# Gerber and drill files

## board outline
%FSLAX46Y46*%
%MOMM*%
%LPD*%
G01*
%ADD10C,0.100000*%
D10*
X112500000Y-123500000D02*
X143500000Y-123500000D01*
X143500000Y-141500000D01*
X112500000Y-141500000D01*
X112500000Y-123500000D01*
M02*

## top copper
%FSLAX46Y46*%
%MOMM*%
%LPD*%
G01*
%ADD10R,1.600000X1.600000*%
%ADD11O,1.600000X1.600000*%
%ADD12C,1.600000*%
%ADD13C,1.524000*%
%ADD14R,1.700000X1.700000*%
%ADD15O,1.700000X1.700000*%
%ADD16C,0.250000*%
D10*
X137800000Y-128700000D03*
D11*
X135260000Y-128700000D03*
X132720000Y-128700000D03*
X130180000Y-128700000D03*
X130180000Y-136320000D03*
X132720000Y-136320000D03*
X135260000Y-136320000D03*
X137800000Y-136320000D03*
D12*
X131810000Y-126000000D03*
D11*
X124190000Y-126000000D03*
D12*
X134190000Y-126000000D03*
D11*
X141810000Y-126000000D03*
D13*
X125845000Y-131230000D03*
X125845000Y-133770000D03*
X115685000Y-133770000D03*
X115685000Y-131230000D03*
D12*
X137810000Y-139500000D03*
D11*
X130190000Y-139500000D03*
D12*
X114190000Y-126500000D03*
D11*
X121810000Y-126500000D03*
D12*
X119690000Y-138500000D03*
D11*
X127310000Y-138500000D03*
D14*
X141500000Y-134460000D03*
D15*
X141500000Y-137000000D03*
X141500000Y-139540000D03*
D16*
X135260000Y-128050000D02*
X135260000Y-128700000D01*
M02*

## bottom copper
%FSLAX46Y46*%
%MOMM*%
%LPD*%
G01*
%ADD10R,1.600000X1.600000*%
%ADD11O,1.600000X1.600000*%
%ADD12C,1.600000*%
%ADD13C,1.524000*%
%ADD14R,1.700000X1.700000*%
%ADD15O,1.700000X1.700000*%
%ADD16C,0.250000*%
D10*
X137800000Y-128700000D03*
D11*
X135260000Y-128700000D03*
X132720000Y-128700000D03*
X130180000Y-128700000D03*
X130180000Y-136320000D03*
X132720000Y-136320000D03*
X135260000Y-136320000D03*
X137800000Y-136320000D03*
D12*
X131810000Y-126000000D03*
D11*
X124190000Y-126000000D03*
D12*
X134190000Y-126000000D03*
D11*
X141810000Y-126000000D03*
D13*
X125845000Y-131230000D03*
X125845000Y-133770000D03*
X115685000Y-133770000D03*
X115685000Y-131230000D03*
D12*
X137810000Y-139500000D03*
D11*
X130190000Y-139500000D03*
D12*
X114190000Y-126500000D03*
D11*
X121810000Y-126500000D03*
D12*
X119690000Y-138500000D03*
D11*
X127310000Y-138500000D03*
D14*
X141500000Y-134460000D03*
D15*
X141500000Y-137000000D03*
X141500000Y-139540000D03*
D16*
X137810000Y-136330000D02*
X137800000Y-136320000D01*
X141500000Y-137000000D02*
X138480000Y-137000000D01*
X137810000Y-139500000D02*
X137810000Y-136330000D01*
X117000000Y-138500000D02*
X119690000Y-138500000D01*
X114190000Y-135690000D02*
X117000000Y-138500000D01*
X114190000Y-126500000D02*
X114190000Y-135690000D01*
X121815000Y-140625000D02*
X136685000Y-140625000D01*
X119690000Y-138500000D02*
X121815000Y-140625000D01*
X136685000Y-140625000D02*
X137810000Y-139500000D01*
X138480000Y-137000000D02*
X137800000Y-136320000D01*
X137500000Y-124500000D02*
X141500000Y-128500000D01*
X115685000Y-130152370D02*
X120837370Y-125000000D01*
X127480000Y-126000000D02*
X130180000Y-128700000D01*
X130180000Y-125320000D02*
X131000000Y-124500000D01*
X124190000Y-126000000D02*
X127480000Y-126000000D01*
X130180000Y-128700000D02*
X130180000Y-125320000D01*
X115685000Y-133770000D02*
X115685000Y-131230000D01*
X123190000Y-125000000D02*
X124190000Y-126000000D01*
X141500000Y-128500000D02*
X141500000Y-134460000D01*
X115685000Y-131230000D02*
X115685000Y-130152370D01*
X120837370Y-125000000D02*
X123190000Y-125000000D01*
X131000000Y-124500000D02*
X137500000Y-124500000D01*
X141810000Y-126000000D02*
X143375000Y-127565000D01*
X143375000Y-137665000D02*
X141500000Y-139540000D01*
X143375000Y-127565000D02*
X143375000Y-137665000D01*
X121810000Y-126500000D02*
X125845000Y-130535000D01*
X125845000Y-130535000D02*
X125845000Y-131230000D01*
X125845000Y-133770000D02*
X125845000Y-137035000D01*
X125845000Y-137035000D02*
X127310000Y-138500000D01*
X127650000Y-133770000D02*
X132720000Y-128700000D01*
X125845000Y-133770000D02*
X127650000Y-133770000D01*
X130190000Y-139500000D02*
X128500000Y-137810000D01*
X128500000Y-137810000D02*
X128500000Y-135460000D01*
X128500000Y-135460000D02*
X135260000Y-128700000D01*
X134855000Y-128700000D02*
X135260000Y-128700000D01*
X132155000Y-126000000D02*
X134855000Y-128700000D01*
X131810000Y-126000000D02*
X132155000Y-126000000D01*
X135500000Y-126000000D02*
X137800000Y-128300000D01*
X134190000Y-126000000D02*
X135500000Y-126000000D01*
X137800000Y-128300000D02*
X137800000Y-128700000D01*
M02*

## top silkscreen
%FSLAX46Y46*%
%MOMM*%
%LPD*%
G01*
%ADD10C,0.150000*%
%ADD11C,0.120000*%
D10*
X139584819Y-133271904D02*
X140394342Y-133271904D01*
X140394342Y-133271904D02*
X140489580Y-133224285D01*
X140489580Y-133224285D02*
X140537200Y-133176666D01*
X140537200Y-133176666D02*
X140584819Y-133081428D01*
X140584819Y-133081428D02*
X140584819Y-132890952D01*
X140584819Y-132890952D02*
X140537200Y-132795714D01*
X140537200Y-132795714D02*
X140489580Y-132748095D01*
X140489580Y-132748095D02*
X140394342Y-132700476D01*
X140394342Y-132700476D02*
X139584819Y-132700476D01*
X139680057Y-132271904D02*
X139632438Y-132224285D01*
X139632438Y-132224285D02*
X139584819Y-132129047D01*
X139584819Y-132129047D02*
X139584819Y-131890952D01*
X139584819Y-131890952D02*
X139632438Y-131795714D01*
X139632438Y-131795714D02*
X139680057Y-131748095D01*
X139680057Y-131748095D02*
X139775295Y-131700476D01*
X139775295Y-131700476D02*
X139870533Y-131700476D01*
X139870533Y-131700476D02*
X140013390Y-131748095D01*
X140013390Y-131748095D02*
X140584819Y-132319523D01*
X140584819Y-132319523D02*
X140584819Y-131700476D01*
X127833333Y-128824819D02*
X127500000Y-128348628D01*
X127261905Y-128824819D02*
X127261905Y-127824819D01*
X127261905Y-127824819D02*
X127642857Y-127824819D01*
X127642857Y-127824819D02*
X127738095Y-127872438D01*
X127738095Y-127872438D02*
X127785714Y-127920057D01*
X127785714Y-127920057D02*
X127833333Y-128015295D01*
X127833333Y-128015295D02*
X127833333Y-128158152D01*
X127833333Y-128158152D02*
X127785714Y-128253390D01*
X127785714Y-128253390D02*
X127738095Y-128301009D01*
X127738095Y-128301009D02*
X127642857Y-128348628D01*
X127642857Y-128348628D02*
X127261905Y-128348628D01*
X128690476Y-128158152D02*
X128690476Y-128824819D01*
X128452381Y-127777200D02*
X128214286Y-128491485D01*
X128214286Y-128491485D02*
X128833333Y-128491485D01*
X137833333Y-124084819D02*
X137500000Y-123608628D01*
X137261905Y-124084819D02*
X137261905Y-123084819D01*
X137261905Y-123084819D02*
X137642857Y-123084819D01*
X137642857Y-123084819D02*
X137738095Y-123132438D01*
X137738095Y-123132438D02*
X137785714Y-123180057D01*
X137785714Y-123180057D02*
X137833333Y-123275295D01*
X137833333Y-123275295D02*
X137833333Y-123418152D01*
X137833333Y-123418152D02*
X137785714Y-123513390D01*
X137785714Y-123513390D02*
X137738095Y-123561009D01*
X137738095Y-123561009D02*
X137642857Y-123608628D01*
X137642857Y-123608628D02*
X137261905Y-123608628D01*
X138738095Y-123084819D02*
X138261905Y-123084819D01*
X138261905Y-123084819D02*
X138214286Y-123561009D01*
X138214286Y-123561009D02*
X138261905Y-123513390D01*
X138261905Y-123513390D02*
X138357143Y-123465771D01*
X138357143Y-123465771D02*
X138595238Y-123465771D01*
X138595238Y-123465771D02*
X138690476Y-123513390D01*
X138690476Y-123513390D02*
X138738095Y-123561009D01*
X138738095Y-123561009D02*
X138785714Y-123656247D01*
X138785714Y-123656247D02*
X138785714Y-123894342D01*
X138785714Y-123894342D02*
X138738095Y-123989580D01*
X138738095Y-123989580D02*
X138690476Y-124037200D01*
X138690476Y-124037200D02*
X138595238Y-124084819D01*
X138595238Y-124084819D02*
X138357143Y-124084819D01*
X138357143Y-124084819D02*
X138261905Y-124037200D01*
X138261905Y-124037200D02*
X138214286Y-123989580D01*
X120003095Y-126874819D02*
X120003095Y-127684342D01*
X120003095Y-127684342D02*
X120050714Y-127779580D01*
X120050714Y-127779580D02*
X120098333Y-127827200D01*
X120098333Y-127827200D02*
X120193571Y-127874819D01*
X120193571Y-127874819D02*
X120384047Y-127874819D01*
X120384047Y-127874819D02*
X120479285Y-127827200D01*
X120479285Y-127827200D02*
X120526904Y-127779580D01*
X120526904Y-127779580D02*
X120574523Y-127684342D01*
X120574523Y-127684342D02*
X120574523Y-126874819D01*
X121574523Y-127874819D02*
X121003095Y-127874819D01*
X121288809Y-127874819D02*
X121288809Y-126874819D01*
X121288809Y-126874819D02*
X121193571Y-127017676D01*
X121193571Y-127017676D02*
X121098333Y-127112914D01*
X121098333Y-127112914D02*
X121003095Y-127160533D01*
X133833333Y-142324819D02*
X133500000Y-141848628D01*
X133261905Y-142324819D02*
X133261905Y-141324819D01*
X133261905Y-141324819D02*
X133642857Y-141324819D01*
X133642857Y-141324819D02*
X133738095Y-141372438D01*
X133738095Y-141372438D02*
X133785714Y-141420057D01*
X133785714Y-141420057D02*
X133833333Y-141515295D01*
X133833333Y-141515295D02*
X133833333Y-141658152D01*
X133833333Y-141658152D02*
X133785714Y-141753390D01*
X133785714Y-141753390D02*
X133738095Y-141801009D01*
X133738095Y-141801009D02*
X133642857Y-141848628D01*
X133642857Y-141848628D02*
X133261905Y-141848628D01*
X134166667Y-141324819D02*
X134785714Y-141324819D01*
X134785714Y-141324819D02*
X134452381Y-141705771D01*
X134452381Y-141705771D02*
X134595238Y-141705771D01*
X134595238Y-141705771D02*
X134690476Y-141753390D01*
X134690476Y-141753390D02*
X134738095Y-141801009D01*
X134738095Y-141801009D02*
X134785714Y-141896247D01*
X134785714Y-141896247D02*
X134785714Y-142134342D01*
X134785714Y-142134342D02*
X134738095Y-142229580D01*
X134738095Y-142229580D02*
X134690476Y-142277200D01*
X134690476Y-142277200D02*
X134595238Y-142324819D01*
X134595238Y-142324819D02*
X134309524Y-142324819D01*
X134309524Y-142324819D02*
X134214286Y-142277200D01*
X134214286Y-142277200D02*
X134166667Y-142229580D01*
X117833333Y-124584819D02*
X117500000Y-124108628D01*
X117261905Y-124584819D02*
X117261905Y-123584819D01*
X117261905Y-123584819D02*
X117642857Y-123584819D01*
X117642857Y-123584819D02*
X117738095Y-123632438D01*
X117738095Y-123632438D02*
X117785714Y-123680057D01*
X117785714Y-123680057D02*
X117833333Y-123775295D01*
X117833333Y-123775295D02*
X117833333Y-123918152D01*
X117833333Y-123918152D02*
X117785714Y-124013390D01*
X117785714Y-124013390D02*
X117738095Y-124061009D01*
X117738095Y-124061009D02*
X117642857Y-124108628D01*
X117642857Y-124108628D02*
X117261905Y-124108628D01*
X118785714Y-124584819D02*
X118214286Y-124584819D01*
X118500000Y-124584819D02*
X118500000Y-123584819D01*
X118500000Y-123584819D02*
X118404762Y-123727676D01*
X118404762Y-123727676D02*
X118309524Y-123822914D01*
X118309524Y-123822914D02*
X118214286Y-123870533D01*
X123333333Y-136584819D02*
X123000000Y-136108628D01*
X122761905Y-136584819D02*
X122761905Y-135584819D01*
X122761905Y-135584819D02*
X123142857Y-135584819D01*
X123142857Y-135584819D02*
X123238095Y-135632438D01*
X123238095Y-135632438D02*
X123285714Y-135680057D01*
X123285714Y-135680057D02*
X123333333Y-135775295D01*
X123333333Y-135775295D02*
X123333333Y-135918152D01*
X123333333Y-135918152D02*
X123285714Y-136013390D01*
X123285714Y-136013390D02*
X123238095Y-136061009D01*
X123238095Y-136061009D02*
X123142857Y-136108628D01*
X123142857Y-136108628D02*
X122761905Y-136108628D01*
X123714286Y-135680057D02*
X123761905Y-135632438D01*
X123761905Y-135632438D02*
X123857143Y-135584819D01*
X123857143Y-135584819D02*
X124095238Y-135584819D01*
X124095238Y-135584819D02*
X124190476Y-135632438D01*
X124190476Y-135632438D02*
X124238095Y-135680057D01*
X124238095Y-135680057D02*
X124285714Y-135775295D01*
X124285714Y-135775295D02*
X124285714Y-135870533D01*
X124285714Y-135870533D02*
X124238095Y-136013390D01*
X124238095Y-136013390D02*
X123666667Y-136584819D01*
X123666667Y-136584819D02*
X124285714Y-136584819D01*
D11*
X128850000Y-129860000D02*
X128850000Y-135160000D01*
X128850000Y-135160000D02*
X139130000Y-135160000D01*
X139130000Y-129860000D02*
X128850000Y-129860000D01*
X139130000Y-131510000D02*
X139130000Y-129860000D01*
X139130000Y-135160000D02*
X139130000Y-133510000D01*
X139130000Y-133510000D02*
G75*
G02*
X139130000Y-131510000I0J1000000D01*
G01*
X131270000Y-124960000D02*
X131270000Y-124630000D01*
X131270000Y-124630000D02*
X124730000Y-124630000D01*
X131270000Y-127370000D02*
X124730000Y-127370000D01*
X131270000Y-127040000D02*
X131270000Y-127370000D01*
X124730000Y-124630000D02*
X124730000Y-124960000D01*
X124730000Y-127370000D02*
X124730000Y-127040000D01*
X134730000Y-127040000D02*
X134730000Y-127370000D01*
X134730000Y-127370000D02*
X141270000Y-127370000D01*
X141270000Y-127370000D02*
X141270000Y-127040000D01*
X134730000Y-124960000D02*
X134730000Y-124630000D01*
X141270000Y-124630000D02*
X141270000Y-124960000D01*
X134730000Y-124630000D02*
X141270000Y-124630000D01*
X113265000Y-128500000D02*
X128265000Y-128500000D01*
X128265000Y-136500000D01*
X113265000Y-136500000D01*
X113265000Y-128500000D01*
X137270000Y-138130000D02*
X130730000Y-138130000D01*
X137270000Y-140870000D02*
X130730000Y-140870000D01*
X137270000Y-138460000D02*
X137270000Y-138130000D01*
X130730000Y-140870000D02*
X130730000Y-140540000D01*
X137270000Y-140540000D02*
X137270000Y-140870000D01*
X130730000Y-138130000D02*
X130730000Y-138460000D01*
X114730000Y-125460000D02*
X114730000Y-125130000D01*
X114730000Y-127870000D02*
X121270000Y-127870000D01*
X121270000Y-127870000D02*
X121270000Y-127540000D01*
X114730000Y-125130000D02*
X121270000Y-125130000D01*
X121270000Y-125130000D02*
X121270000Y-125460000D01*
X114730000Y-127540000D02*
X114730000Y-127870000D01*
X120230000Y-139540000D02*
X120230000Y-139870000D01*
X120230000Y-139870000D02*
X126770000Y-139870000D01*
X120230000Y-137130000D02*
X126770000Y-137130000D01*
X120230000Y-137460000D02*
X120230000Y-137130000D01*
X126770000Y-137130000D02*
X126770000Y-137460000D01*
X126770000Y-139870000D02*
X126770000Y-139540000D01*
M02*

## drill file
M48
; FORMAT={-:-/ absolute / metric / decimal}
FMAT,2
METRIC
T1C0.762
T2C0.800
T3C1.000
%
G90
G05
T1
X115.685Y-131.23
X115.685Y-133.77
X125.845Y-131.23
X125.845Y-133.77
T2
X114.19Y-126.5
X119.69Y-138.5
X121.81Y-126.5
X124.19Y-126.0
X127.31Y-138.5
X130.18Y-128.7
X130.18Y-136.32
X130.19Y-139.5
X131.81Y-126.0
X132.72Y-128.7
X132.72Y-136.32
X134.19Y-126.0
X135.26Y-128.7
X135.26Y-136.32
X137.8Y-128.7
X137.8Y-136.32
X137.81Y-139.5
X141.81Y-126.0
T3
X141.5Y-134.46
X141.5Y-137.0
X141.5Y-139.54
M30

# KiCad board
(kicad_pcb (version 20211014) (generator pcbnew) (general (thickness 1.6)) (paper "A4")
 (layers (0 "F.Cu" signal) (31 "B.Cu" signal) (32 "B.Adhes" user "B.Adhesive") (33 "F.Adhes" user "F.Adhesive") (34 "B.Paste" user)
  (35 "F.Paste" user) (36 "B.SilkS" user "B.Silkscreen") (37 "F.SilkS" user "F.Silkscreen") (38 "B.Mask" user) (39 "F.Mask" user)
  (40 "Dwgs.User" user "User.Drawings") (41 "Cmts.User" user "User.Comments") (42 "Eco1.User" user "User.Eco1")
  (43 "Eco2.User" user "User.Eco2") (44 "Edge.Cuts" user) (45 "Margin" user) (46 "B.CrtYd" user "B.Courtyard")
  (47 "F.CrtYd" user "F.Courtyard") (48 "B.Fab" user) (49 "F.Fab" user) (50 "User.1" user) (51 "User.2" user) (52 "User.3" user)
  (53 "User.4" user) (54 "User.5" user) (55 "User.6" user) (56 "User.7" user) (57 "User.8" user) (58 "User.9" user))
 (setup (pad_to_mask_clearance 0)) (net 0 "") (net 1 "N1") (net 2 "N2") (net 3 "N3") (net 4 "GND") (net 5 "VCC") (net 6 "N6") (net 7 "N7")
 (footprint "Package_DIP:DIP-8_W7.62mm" (layer "F.Cu") (at 137.8 128.7 -90)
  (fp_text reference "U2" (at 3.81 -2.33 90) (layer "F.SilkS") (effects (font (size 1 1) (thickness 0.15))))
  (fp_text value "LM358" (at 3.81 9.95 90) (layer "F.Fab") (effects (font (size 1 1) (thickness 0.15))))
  (fp_line (start 1.16 8.95) (end 6.46 8.95) (layer "F.SilkS") (width 0.12))
  (fp_line (start 6.46 8.95) (end 6.46 -1.33) (layer "F.SilkS") (width 0.12))
  (fp_line (start 1.16 -1.33) (end 1.16 8.95) (layer "F.SilkS") (width 0.12))
  (fp_line (start 2.81 -1.33) (end 1.16 -1.33) (layer "F.SilkS") (width 0.12))
  (fp_line (start 6.46 -1.33) (end 4.81 -1.33) (layer "F.SilkS") (width 0.12))
  (fp_arc (start 4.81 -1.33) (mid 3.81 -0.33) (end 2.81 -1.33) (layer "F.SilkS") (width 0.12))
  (pad "1" thru_hole rect (at 0 0 270) (size 1.6 1.6) (drill 0.8) (layers *.Cu *.Mask) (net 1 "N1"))
  (pad "2" thru_hole oval (at 0 2.54 270) (size 1.6 1.6) (drill 0.8) (layers *.Cu *.Mask) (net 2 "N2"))
  (pad "3" thru_hole oval (at 0 5.08 270) (size 1.6 1.6) (drill 0.8) (layers *.Cu *.Mask) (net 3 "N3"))
  (pad "4" thru_hole oval (at 0 7.62 270) (size 1.6 1.6) (drill 0.8) (layers *.Cu *.Mask) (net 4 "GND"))
  (pad "5" thru_hole oval (at 7.62 7.62 270) (size 1.6 1.6) (drill 0.8) (layers *.Cu *.Mask))
  (pad "6" thru_hole oval (at 7.62 5.08 270) (size 1.6 1.6) (drill 0.8) (layers *.Cu *.Mask))
  (pad "7" thru_hole oval (at 7.62 2.54 270) (size 1.6 1.6) (drill 0.8) (layers *.Cu *.Mask))
  (pad "8" thru_hole oval (at 7.62 0 270) (size 1.6 1.6) (drill 0.8) (layers *.Cu *.Mask) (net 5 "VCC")))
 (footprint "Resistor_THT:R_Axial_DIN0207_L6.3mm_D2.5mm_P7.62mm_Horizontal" (layer "F.Cu") (at 131.81 126 180)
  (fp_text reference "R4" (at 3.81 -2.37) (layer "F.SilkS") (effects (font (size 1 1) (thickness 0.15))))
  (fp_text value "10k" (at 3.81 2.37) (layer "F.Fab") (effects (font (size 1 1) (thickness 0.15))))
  (fp_line (start 0.54 1.04) (end 0.54 1.37) (layer "F.SilkS") (width 0.12))
  (fp_line (start 0.54 1.37) (end 7.08 1.37) (layer "F.SilkS") (width 0.12))
  (fp_line (start 0.54 -1.37) (end 7.08 -1.37) (layer "F.SilkS") (width 0.12))
  (fp_line (start 0.54 -1.04) (end 0.54 -1.37) (layer "F.SilkS") (width 0.12))
  (fp_line (start 7.08 1.37) (end 7.08 1.04) (layer "F.SilkS") (width 0.12))
  (fp_line (start 7.08 -1.37) (end 7.08 -1.04) (layer "F.SilkS") (width 0.12))
  (pad "1" thru_hole circle (at 0 0 180) (size 1.6 1.6) (drill 0.8) (layers *.Cu *.Mask) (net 2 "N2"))
  (pad "2" thru_hole oval (at 7.62 0 180) (size 1.6 1.6) (drill 0.8) (layers *.Cu *.Mask) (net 4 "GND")))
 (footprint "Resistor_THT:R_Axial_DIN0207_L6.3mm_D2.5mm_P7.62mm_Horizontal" (layer "F.Cu") (at 134.19 126)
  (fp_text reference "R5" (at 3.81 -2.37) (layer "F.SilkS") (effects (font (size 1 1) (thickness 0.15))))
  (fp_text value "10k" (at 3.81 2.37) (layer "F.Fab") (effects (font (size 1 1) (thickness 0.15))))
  (fp_line (start 0.54 1.04) (end 0.54 1.37) (layer "F.SilkS") (width 0.12))
  (fp_line (start 0.54 1.37) (end 7.08 1.37) (layer "F.SilkS") (width 0.12))
  (fp_line (start 7.08 1.37) (end 7.08 1.04) (layer "F.SilkS") (width 0.12))
  (fp_line (start 0.54 -1.04) (end 0.54 -1.37) (layer "F.SilkS") (width 0.12))
  (fp_line (start 7.08 -1.37) (end 7.08 -1.04) (layer "F.SilkS") (width 0.12))
  (fp_line (start 0.54 -1.37) (end 7.08 -1.37) (layer "F.SilkS") (width 0.12))
  (pad "1" thru_hole circle (at 0 0) (size 1.6 1.6) (drill 0.8) (layers *.Cu *.Mask) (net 1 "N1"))
  (pad "2" thru_hole oval (at 7.62 0) (size 1.6 1.6) (drill 0.8) (layers *.Cu *.Mask) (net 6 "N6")))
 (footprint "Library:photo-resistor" (layer "F.Cu") (at 120.765 132.5)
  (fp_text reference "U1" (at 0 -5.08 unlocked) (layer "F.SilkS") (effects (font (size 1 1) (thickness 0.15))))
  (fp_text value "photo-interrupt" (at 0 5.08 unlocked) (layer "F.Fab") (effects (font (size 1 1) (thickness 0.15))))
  (fp_rect (start 7.5 -4) (end -7.5 4) (layer "F.SilkS") (width 0.12) (fill none))
  (pad "1" thru_hole circle (at 5.08 -1.27) (size 1.524 1.524) (drill 0.762) (layers *.Cu *.Mask) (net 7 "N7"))
  (pad "2" thru_hole circle (at 5.08 1.27) (size 1.524 1.524) (drill 0.762) (layers *.Cu *.Mask) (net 3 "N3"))
  (pad "3" thru_hole circle (at -5.08 1.27) (size 1.524 1.524) (drill 0.762) (layers *.Cu *.Mask) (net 4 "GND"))
  (pad "4" thru_hole circle (at -5.08 -1.27) (size 1.524 1.524) (drill 0.762) (layers *.Cu *.Mask) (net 4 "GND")))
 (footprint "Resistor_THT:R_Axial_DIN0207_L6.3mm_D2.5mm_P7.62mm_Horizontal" (layer "F.Cu") (at 137.81 139.5 180)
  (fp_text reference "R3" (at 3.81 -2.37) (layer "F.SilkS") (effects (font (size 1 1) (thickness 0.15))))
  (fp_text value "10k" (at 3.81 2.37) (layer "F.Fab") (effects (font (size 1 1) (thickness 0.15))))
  (fp_line (start 0.54 1.37) (end 7.08 1.37) (layer "F.SilkS") (width 0.12))
  (fp_line (start 0.54 -1.37) (end 7.08 -1.37) (layer "F.SilkS") (width 0.12))
  (fp_line (start 0.54 1.04) (end 0.54 1.37) (layer "F.SilkS") (width 0.12))
  (fp_line (start 7.08 -1.37) (end 7.08 -1.04) (layer "F.SilkS") (width 0.12))
  (fp_line (start 0.54 -1.04) (end 0.54 -1.37) (layer "F.SilkS") (width 0.12))
  (fp_line (start 7.08 1.37) (end 7.08 1.04) (layer "F.SilkS") (width 0.12))
  (pad "1" thru_hole circle (at 0 0 180) (size 1.6 1.6) (drill 0.8) (layers *.Cu *.Mask) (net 5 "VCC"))
  (pad "2" thru_hole oval (at 7.62 0 180) (size 1.6 1.6) (drill 0.8) (layers *.Cu *.Mask) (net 2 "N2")))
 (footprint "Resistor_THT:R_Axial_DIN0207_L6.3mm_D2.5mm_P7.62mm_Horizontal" (layer "F.Cu") (at 114.19 126.5)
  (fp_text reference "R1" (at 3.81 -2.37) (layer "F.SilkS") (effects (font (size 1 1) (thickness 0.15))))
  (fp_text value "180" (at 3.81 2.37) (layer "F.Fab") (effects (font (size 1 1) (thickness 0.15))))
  (fp_line (start 0.54 -1.04) (end 0.54 -1.37) (layer "F.SilkS") (width 0.12))
  (fp_line (start 0.54 1.37) (end 7.08 1.37) (layer "F.SilkS") (width 0.12))
  (fp_line (start 7.08 1.37) (end 7.08 1.04) (layer "F.SilkS") (width 0.12))
  (fp_line (start 0.54 -1.37) (end 7.08 -1.37) (layer "F.SilkS") (width 0.12))
  (fp_line (start 7.08 -1.37) (end 7.08 -1.04) (layer "F.SilkS") (width 0.12))
  (fp_line (start 0.54 1.04) (end 0.54 1.37) (layer "F.SilkS") (width 0.12))
  (pad "1" thru_hole circle (at 0 0) (size 1.6 1.6) (drill 0.8) (layers *.Cu *.Mask) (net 5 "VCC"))
  (pad "2" thru_hole oval (at 7.62 0) (size 1.6 1.6) (drill 0.8) (layers *.Cu *.Mask) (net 7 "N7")))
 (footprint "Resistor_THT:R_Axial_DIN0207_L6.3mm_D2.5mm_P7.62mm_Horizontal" (layer "F.Cu") (at 119.69 138.5)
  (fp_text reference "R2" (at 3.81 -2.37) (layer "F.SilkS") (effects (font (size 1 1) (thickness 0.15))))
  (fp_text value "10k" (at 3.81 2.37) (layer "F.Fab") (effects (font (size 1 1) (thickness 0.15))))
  (fp_line (start 0.54 1.04) (end 0.54 1.37) (layer "F.SilkS") (width 0.12))
  (fp_line (start 0.54 1.37) (end 7.08 1.37) (layer "F.SilkS") (width 0.12))
  (fp_line (start 0.54 -1.37) (end 7.08 -1.37) (layer "F.SilkS") (width 0.12))
  (fp_line (start 0.54 -1.04) (end 0.54 -1.37) (layer "F.SilkS") (width 0.12))
  (fp_line (start 7.08 -1.37) (end 7.08 -1.04) (layer "F.SilkS") (width 0.12))
  (fp_line (start 7.08 1.37) (end 7.08 1.04) (layer "F.SilkS") (width 0.12))
  (pad "1" thru_hole circle (at 0 0) (size 1.6 1.6) (drill 0.8) (layers *.Cu *.Mask) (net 5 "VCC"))
  (pad "2" thru_hole oval (at 7.62 0) (size 1.6 1.6) (drill 0.8) (layers *.Cu *.Mask) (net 3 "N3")))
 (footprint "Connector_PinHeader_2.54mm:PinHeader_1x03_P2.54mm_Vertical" (layer "B.Cu") (at 141.5 134.46 180)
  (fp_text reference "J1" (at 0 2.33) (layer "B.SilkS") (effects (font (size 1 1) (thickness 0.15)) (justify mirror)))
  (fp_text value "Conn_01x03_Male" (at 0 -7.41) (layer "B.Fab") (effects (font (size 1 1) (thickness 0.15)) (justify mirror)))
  (pad "1" thru_hole rect (at 0 0 180) (size 1.7 1.7) (drill 1) (layers *.Cu *.Mask) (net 4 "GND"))
  (pad "2" thru_hole oval (at 0 -2.54 180) (size 1.7 1.7) (drill 1) (layers *.Cu *.Mask) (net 5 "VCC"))
  (pad "3" thru_hole oval (at 0 -5.08 180) (size 1.7 1.7) (drill 1) (layers *.Cu *.Mask) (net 6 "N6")))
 (gr_rect (start 143.5 123.5) (end 112.5 141.5) (layer "Edge.Cuts") (width 0.1) (fill none))
 (segment (start 137.81 136.33) (end 137.8 136.32) (width 0.25) (layer "B.Cu") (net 5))
 (segment (start 141.5 137) (end 138.48 137) (width 0.25) (layer "B.Cu") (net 5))
 (segment (start 137.81 139.5) (end 137.81 136.33) (width 0.25) (layer "B.Cu") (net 5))
 (segment (start 117 138.5) (end 119.69 138.5) (width 0.25) (layer "B.Cu") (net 5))
 (segment (start 114.19 135.69) (end 117 138.5) (width 0.25) (layer "B.Cu") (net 5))
 (segment (start 114.19 126.5) (end 114.19 135.69) (width 0.25) (layer "B.Cu") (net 5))
 (segment (start 121.815 140.625) (end 136.685 140.625) (width 0.25) (layer "B.Cu") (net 5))
 (segment (start 119.69 138.5) (end 121.815 140.625) (width 0.25) (layer "B.Cu") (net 5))
 (segment (start 136.685 140.625) (end 137.81 139.5) (width 0.25) (layer "B.Cu") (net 5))
 (segment (start 138.48 137) (end 137.8 136.32) (width 0.25) (layer "B.Cu") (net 5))
 (segment (start 137.5 124.5) (end 141.5 128.5) (width 0.25) (layer "B.Cu") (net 4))
 (segment (start 115.685 130.15237) (end 120.83737 125) (width 0.25) (layer "B.Cu") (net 4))
 (segment (start 127.48 126) (end 130.18 128.7) (width 0.25) (layer "B.Cu") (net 4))
 (segment (start 130.18 125.32) (end 131 124.5) (width 0.25) (layer "B.Cu") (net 4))
 (segment (start 124.19 126) (end 127.48 126) (width 0.25) (layer "B.Cu") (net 4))
 (segment (start 130.18 128.7) (end 130.18 125.32) (width 0.25) (layer "B.Cu") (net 4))
 (segment (start 115.685 133.77) (end 115.685 131.23) (width 0.25) (layer "B.Cu") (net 4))
 (segment (start 123.19 125) (end 124.19 126) (width 0.25) (layer "B.Cu") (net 4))
 (segment (start 141.5 128.5) (end 141.5 134.46) (width 0.25) (layer "B.Cu") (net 4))
 (segment (start 115.685 131.23) (end 115.685 130.15237) (width 0.25) (layer "B.Cu") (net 4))
 (segment (start 120.83737 125) (end 123.19 125) (width 0.25) (layer "B.Cu") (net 4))
 (segment (start 131 124.5) (end 137.5 124.5) (width 0.25) (layer "B.Cu") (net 4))
 (segment (start 141.81 126) (end 143.375 127.565) (width 0.25) (layer "B.Cu") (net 6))
 (segment (start 143.375 137.665) (end 141.5 139.54) (width 0.25) (layer "B.Cu") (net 6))
 (segment (start 143.375 127.565) (end 143.375 137.665) (width 0.25) (layer "B.Cu") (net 6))
 (segment (start 121.81 126.5) (end 125.845 130.535) (width 0.25) (layer "B.Cu") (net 7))
 (segment (start 125.845 130.535) (end 125.845 131.23) (width 0.25) (layer "B.Cu") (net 7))
 (segment (start 125.845 133.77) (end 125.845 137.035) (width 0.25) (layer "B.Cu") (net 3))
 (segment (start 125.845 137.035) (end 127.31 138.5) (width 0.25) (layer "B.Cu") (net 3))
 (segment (start 127.65 133.77) (end 132.72 128.7) (width 0.25) (layer "B.Cu") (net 3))
 (segment (start 125.845 133.77) (end 127.65 133.77) (width 0.25) (layer "B.Cu") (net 3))
 (segment (start 135.26 128.05) (end 135.26 128.7) (width 0.25) (layer "F.Cu") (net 2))
 (segment (start 130.19 139.5) (end 128.5 137.81) (width 0.25) (layer "B.Cu") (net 2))
 (segment (start 128.5 137.81) (end 128.5 135.46) (width 0.25) (layer "B.Cu") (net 2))
 (segment (start 128.5 135.46) (end 135.26 128.7) (width 0.25) (layer "B.Cu") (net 2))
 (segment (start 134.855 128.7) (end 135.26 128.7) (width 0.25) (layer "B.Cu") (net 2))
 (segment (start 132.155 126) (end 134.855 128.7) (width 0.25) (layer "B.Cu") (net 2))
 (segment (start 131.81 126) (end 132.155 126) (width 0.25) (layer "B.Cu") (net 2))
 (segment (start 135.5 126) (end 137.8 128.3) (width 0.25) (layer "B.Cu") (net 1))
 (segment (start 134.19 126) (end 135.5 126) (width 0.25) (layer "B.Cu") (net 1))
 (segment (start 137.8 128.3) (end 137.8 128.7) (width 0.25) (layer "B.Cu") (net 1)))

